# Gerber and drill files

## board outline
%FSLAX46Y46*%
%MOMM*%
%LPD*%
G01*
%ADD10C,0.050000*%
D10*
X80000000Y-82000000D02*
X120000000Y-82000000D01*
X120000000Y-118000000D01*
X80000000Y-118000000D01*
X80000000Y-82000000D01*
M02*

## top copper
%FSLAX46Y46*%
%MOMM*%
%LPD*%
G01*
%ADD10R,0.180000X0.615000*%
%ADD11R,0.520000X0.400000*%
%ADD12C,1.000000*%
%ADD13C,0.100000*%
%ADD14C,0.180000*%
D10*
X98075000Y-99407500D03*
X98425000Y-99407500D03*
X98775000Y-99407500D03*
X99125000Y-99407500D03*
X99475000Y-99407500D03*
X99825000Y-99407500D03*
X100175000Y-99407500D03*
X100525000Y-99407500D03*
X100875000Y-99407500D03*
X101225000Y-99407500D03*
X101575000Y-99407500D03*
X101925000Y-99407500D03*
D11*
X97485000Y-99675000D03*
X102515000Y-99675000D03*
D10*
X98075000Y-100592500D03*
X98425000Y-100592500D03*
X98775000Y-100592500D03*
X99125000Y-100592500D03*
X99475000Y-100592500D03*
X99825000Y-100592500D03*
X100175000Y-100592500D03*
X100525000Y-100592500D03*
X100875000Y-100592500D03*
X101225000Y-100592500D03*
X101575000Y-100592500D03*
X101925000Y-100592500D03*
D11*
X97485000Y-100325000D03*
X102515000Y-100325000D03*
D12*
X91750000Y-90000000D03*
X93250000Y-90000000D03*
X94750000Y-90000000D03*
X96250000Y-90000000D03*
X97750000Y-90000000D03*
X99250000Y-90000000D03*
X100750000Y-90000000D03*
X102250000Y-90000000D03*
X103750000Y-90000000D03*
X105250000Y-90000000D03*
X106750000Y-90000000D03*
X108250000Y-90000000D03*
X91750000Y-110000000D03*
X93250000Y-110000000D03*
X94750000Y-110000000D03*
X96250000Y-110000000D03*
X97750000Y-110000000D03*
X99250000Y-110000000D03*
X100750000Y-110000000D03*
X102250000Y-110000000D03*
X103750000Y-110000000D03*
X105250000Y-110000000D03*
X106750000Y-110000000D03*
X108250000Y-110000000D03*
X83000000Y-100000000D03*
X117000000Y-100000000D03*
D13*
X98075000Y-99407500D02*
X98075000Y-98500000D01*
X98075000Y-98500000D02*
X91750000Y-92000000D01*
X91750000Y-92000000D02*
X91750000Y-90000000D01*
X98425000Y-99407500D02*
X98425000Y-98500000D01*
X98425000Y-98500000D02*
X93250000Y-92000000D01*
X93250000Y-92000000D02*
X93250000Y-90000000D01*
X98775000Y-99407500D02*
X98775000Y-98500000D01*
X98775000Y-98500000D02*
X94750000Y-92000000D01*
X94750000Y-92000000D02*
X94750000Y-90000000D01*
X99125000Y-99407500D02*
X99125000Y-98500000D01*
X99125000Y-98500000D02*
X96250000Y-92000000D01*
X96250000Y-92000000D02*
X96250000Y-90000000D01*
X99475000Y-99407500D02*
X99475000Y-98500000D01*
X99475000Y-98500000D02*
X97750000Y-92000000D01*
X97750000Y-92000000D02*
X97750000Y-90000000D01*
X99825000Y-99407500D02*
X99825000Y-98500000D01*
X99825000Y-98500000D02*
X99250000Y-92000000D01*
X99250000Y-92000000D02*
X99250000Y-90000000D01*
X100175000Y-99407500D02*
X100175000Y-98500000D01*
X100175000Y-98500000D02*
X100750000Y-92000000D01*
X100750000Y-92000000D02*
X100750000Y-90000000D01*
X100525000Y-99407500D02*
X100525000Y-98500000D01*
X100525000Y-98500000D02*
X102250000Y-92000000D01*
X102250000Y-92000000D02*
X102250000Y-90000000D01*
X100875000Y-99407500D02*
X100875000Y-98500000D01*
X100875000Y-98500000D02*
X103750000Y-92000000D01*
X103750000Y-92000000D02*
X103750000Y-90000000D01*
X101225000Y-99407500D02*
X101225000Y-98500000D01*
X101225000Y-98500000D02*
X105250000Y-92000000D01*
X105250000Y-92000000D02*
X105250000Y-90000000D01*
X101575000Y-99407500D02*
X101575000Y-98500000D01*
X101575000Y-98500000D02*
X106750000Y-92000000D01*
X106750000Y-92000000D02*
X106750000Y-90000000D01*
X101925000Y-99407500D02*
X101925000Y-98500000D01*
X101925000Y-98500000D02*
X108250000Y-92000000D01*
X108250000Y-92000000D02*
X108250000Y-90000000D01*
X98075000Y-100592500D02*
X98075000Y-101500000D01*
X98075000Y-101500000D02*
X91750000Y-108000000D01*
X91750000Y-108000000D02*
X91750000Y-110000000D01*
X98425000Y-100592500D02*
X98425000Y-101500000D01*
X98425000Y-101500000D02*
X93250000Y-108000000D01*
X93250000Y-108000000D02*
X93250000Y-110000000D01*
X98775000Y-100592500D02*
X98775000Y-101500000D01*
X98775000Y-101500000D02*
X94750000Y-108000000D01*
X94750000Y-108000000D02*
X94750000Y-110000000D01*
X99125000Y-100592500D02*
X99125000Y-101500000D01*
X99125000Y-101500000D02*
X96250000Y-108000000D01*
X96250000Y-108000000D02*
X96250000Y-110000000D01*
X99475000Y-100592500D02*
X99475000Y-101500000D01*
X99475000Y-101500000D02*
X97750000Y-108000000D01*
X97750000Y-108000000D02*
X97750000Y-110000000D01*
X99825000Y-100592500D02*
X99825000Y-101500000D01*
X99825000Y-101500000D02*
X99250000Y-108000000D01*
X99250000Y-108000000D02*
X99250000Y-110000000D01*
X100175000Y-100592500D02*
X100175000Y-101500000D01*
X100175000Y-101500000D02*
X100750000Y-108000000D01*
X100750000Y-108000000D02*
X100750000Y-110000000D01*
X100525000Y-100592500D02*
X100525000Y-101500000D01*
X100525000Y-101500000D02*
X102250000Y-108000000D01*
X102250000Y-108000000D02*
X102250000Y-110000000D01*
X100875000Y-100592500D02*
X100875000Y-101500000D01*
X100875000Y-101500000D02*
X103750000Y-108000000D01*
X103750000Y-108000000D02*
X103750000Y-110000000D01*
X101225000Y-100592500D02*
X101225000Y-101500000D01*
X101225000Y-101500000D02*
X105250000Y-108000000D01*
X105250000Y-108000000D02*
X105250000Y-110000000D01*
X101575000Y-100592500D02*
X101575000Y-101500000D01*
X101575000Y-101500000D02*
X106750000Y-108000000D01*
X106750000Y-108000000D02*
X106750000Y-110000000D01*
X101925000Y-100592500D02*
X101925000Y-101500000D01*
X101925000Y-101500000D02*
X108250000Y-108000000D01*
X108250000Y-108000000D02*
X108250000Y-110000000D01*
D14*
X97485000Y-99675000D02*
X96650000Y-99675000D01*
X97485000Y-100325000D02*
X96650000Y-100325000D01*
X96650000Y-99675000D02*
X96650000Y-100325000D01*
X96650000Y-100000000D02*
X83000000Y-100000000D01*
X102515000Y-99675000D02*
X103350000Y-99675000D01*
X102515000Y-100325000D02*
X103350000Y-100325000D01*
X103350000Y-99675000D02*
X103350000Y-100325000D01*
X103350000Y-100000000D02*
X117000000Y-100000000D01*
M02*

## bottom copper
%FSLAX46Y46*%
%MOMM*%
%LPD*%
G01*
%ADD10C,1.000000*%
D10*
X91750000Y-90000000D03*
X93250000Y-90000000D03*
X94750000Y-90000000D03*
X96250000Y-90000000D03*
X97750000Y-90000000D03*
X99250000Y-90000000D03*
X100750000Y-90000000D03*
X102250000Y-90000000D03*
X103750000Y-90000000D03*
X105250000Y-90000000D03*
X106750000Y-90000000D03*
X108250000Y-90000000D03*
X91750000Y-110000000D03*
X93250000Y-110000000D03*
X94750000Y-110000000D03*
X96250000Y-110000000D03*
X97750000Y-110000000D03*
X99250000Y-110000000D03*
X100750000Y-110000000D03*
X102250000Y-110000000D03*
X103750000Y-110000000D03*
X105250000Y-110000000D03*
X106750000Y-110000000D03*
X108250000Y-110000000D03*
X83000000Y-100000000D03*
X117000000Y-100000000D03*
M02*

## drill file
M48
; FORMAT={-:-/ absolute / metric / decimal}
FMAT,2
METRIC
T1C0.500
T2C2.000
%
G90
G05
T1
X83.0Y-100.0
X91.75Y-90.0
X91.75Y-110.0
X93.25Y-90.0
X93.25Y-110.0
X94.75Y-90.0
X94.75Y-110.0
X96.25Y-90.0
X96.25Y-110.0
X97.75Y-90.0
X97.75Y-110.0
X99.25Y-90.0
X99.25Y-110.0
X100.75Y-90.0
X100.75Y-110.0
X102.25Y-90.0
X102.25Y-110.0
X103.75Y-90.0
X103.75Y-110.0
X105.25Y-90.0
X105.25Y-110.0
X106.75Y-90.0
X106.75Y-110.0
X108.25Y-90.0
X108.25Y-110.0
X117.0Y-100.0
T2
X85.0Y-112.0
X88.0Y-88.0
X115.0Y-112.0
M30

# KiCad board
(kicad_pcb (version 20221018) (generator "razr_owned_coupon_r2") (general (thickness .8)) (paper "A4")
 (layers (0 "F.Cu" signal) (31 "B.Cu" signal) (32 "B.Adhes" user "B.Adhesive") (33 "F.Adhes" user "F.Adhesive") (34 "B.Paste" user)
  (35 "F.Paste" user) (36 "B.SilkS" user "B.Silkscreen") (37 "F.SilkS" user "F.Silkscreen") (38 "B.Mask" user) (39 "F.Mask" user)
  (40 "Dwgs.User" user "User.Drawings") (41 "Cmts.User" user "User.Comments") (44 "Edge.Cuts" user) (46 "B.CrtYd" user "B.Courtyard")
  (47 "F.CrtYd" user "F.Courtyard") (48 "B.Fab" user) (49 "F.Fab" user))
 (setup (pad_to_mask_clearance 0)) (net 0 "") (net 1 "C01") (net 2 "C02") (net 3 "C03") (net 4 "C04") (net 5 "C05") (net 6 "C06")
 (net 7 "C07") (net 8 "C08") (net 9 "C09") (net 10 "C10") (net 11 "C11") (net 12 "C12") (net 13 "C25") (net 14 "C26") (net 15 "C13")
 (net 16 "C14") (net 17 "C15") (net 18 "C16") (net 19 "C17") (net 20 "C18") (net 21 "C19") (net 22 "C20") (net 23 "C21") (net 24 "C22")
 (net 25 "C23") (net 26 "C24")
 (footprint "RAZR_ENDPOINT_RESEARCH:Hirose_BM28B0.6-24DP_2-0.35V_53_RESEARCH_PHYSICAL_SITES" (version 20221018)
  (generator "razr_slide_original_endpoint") (layer "F.Cu") (at 100 100)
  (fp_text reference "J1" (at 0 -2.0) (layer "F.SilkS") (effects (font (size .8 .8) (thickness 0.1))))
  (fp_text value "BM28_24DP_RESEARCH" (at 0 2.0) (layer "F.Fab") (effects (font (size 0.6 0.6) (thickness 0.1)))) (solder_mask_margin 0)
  (pad "S_NEG_00" smd rect (at -1.925 -0.5925) (size 0.18 0.615) (layers "F.Cu" "F.Mask") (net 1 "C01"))
  (pad "S_NEG_01" smd rect (at -1.575 -0.5925) (size 0.18 0.615) (layers "F.Cu" "F.Mask") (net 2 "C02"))
  (pad "S_NEG_02" smd rect (at -1.225 -0.5925) (size 0.18 0.615) (layers "F.Cu" "F.Mask") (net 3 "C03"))
  (pad "S_NEG_03" smd rect (at -0.875 -0.5925) (size 0.18 0.615) (layers "F.Cu" "F.Mask") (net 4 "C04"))
  (pad "S_NEG_04" smd rect (at -0.525 -0.5925) (size 0.18 0.615) (layers "F.Cu" "F.Mask") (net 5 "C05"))
  (pad "S_NEG_05" smd rect (at -0.175 -0.5925) (size 0.18 0.615) (layers "F.Cu" "F.Mask") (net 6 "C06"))
  (pad "S_NEG_06" smd rect (at 0.175 -0.5925) (size 0.18 0.615) (layers "F.Cu" "F.Mask") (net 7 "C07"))
  (pad "S_NEG_07" smd rect (at 0.525 -0.5925) (size 0.18 0.615) (layers "F.Cu" "F.Mask") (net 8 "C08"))
  (pad "S_NEG_08" smd rect (at 0.875 -0.5925) (size 0.18 0.615) (layers "F.Cu" "F.Mask") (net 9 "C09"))
  (pad "S_NEG_09" smd rect (at 1.225 -0.5925) (size 0.18 0.615) (layers "F.Cu" "F.Mask") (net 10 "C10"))
  (pad "S_NEG_10" smd rect (at 1.575 -0.5925) (size 0.18 0.615) (layers "F.Cu" "F.Mask") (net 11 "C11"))
  (pad "S_NEG_11" smd rect (at 1.925 -0.5925) (size 0.18 0.615) (layers "F.Cu" "F.Mask") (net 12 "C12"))
  (pad "P_L" smd rect (at -2.515 -0.325) (size 0.52 0.4) (layers "F.Cu" "F.Mask") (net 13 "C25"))
  (pad "P_R" smd rect (at 2.515 -0.325) (size 0.52 0.4) (layers "F.Cu" "F.Mask") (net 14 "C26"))
  (pad "S_POS_00" smd rect (at -1.925 0.5925) (size 0.18 0.615) (layers "F.Cu" "F.Mask") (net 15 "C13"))
  (pad "S_POS_01" smd rect (at -1.575 0.5925) (size 0.18 0.615) (layers "F.Cu" "F.Mask") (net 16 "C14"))
  (pad "S_POS_02" smd rect (at -1.225 0.5925) (size 0.18 0.615) (layers "F.Cu" "F.Mask") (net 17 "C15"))
  (pad "S_POS_03" smd rect (at -0.875 0.5925) (size 0.18 0.615) (layers "F.Cu" "F.Mask") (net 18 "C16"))
  (pad "S_POS_04" smd rect (at -0.525 0.5925) (size 0.18 0.615) (layers "F.Cu" "F.Mask") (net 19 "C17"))
  (pad "S_POS_05" smd rect (at -0.175 0.5925) (size 0.18 0.615) (layers "F.Cu" "F.Mask") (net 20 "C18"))
  (pad "S_POS_06" smd rect (at 0.175 0.5925) (size 0.18 0.615) (layers "F.Cu" "F.Mask") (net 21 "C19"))
  (pad "S_POS_07" smd rect (at 0.525 0.5925) (size 0.18 0.615) (layers "F.Cu" "F.Mask") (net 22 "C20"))
  (pad "S_POS_08" smd rect (at 0.875 0.5925) (size 0.18 0.615) (layers "F.Cu" "F.Mask") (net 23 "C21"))
  (pad "S_POS_09" smd rect (at 1.225 0.5925) (size 0.18 0.615) (layers "F.Cu" "F.Mask") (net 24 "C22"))
  (pad "S_POS_10" smd rect (at 1.575 0.5925) (size 0.18 0.615) (layers "F.Cu" "F.Mask") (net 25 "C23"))
  (pad "S_POS_11" smd rect (at 1.925 0.5925) (size 0.18 0.615) (layers "F.Cu" "F.Mask") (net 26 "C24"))
  (pad "P_L" smd rect (at -2.515 0.325) (size 0.52 0.4) (layers "F.Cu" "F.Mask") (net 13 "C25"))
  (pad "P_R" smd rect (at 2.515 0.325) (size 0.52 0.4) (layers "F.Cu" "F.Mask") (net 14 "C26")))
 (segment (start 98.075000 99.407500) (end 98.075000 98.500000) (width 0.1) (layer "F.Cu") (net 1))
 (segment (start 98.075000 98.500000) (end 91.750000 92.000000) (width 0.1) (layer "F.Cu") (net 1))
 (segment (start 91.750000 92.000000) (end 91.750000 90.000000) (width 0.1) (layer "F.Cu") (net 1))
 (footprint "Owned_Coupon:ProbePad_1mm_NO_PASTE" (layer "F.Cu") (at 91.75 90)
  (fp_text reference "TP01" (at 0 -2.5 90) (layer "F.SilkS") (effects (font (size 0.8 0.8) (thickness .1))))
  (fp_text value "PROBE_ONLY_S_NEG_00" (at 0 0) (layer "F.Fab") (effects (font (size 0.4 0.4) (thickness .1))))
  (pad "1" thru_hole circle (at 0 0) (size 1 1) (drill .5) (layers "*.Cu" "*.Mask") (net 1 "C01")))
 (segment (start 98.425000 99.407500) (end 98.425000 98.500000) (width 0.1) (layer "F.Cu") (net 2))
 (segment (start 98.425000 98.500000) (end 93.250000 92.000000) (width 0.1) (layer "F.Cu") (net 2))
 (segment (start 93.250000 92.000000) (end 93.250000 90.000000) (width 0.1) (layer "F.Cu") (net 2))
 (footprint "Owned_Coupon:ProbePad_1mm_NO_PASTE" (layer "F.Cu") (at 93.25 90)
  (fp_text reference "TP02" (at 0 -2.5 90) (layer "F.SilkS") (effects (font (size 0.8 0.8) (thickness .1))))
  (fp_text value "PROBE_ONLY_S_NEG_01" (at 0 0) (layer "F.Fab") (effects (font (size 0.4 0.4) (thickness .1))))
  (pad "1" thru_hole circle (at 0 0) (size 1 1) (drill .5) (layers "*.Cu" "*.Mask") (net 2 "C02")))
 (segment (start 98.775000 99.407500) (end 98.775000 98.500000) (width 0.1) (layer "F.Cu") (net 3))
 (segment (start 98.775000 98.500000) (end 94.750000 92.000000) (width 0.1) (layer "F.Cu") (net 3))
 (segment (start 94.750000 92.000000) (end 94.750000 90.000000) (width 0.1) (layer "F.Cu") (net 3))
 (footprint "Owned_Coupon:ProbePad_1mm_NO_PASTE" (layer "F.Cu") (at 94.75 90)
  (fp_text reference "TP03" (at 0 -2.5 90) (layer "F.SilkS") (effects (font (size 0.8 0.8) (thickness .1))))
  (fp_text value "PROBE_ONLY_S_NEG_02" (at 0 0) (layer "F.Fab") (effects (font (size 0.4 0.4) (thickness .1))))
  (pad "1" thru_hole circle (at 0 0) (size 1 1) (drill .5) (layers "*.Cu" "*.Mask") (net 3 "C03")))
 (segment (start 99.125000 99.407500) (end 99.125000 98.500000) (width 0.1) (layer "F.Cu") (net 4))
 (segment (start 99.125000 98.500000) (end 96.250000 92.000000) (width 0.1) (layer "F.Cu") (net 4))
 (segment (start 96.250000 92.000000) (end 96.250000 90.000000) (width 0.1) (layer "F.Cu") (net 4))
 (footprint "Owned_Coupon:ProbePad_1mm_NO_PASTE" (layer "F.Cu") (at 96.25 90)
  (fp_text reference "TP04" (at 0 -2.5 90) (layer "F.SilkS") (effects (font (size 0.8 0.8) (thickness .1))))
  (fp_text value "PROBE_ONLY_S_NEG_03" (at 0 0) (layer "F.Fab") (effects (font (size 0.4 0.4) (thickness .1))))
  (pad "1" thru_hole circle (at 0 0) (size 1 1) (drill .5) (layers "*.Cu" "*.Mask") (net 4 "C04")))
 (segment (start 99.475000 99.407500) (end 99.475000 98.500000) (width 0.1) (layer "F.Cu") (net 5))
 (segment (start 99.475000 98.500000) (end 97.750000 92.000000) (width 0.1) (layer "F.Cu") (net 5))
 (segment (start 97.750000 92.000000) (end 97.750000 90.000000) (width 0.1) (layer "F.Cu") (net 5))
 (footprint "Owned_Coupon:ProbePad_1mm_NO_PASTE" (layer "F.Cu") (at 97.75 90)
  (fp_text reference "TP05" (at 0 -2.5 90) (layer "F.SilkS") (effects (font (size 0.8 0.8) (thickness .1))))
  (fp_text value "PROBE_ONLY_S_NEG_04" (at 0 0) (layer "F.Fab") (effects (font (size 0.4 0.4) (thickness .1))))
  (pad "1" thru_hole circle (at 0 0) (size 1 1) (drill .5) (layers "*.Cu" "*.Mask") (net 5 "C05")))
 (segment (start 99.825000 99.407500) (end 99.825000 98.500000) (width 0.1) (layer "F.Cu") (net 6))
 (segment (start 99.825000 98.500000) (end 99.250000 92.000000) (width 0.1) (layer "F.Cu") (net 6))
 (segment (start 99.250000 92.000000) (end 99.250000 90.000000) (width 0.1) (layer "F.Cu") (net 6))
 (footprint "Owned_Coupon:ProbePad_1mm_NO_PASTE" (layer "F.Cu") (at 99.25 90)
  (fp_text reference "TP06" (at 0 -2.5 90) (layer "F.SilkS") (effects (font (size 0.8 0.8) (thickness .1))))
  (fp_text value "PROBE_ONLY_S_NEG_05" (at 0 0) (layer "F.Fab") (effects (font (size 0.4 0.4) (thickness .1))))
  (pad "1" thru_hole circle (at 0 0) (size 1 1) (drill .5) (layers "*.Cu" "*.Mask") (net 6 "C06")))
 (segment (start 100.175000 99.407500) (end 100.175000 98.500000) (width 0.1) (layer "F.Cu") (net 7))
 (segment (start 100.175000 98.500000) (end 100.750000 92.000000) (width 0.1) (layer "F.Cu") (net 7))
 (segment (start 100.750000 92.000000) (end 100.750000 90.000000) (width 0.1) (layer "F.Cu") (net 7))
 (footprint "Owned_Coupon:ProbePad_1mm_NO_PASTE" (layer "F.Cu") (at 100.75 90)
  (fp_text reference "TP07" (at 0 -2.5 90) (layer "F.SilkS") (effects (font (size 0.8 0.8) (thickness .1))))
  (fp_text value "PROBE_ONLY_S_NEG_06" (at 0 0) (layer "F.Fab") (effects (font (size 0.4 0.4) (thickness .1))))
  (pad "1" thru_hole circle (at 0 0) (size 1 1) (drill .5) (layers "*.Cu" "*.Mask") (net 7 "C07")))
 (segment (start 100.525000 99.407500) (end 100.525000 98.500000) (width 0.1) (layer "F.Cu") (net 8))
 (segment (start 100.525000 98.500000) (end 102.250000 92.000000) (width 0.1) (layer "F.Cu") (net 8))
 (segment (start 102.250000 92.000000) (end 102.250000 90.000000) (width 0.1) (layer "F.Cu") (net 8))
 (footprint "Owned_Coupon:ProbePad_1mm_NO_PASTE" (layer "F.Cu") (at 102.25 90)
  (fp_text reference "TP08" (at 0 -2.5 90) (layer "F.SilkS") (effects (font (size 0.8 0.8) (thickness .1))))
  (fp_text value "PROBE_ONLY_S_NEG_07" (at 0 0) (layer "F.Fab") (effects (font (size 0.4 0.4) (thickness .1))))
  (pad "1" thru_hole circle (at 0 0) (size 1 1) (drill .5) (layers "*.Cu" "*.Mask") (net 8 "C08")))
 (segment (start 100.875000 99.407500) (end 100.875000 98.500000) (width 0.1) (layer "F.Cu") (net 9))
 (segment (start 100.875000 98.500000) (end 103.750000 92.000000) (width 0.1) (layer "F.Cu") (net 9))
 (segment (start 103.750000 92.000000) (end 103.750000 90.000000) (width 0.1) (layer "F.Cu") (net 9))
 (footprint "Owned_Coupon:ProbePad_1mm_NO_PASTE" (layer "F.Cu") (at 103.75 90)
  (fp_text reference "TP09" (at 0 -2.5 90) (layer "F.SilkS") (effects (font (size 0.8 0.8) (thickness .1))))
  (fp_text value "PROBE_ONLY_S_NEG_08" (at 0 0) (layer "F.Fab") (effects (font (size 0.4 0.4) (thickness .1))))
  (pad "1" thru_hole circle (at 0 0) (size 1 1) (drill .5) (layers "*.Cu" "*.Mask") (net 9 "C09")))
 (segment (start 101.225000 99.407500) (end 101.225000 98.500000) (width 0.1) (layer "F.Cu") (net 10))
 (segment (start 101.225000 98.500000) (end 105.250000 92.000000) (width 0.1) (layer "F.Cu") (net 10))
 (segment (start 105.250000 92.000000) (end 105.250000 90.000000) (width 0.1) (layer "F.Cu") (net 10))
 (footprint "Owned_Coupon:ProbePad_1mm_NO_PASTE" (layer "F.Cu") (at 105.25 90)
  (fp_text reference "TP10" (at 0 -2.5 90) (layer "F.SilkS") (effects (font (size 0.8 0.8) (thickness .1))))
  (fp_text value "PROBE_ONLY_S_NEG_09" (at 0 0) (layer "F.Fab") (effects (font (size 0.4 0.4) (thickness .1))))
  (pad "1" thru_hole circle (at 0 0) (size 1 1) (drill .5) (layers "*.Cu" "*.Mask") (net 10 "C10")))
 (segment (start 101.575000 99.407500) (end 101.575000 98.500000) (width 0.1) (layer "F.Cu") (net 11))
 (segment (start 101.575000 98.500000) (end 106.750000 92.000000) (width 0.1) (layer "F.Cu") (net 11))
 (segment (start 106.750000 92.000000) (end 106.750000 90.000000) (width 0.1) (layer "F.Cu") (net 11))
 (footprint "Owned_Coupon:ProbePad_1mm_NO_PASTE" (layer "F.Cu") (at 106.75 90)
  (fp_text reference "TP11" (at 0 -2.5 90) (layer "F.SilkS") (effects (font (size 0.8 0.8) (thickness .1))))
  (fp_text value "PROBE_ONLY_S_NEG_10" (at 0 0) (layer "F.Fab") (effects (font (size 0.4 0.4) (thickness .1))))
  (pad "1" thru_hole circle (at 0 0) (size 1 1) (drill .5) (layers "*.Cu" "*.Mask") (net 11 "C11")))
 (segment (start 101.925000 99.407500) (end 101.925000 98.500000) (width 0.1) (layer "F.Cu") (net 12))
 (segment (start 101.925000 98.500000) (end 108.250000 92.000000) (width 0.1) (layer "F.Cu") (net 12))
 (segment (start 108.250000 92.000000) (end 108.250000 90.000000) (width 0.1) (layer "F.Cu") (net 12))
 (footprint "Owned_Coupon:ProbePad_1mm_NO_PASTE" (layer "F.Cu") (at 108.25 90)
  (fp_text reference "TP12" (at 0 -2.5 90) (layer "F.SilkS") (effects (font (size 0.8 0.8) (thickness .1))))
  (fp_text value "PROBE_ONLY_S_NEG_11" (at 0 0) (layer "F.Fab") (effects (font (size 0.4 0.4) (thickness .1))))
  (pad "1" thru_hole circle (at 0 0) (size 1 1) (drill .5) (layers "*.Cu" "*.Mask") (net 12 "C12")))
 (segment (start 98.075000 100.592500) (end 98.075000 101.500000) (width 0.1) (layer "F.Cu") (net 15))
 (segment (start 98.075000 101.500000) (end 91.750000 108.000000) (width 0.1) (layer "F.Cu") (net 15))
 (segment (start 91.750000 108.000000) (end 91.750000 110.000000) (width 0.1) (layer "F.Cu") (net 15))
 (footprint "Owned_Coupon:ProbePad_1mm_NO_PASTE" (layer "F.Cu") (at 91.75 110)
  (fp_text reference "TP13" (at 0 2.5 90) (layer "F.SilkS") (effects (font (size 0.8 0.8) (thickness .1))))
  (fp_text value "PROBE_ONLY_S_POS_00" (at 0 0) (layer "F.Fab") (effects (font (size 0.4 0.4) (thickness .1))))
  (pad "1" thru_hole circle (at 0 0) (size 1 1) (drill .5) (layers "*.Cu" "*.Mask") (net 15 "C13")))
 (segment (start 98.425000 100.592500) (end 98.425000 101.500000) (width 0.1) (layer "F.Cu") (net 16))
 (segment (start 98.425000 101.500000) (end 93.250000 108.000000) (width 0.1) (layer "F.Cu") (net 16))
 (segment (start 93.250000 108.000000) (end 93.250000 110.000000) (width 0.1) (layer "F.Cu") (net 16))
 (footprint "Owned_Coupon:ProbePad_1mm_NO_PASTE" (layer "F.Cu") (at 93.25 110)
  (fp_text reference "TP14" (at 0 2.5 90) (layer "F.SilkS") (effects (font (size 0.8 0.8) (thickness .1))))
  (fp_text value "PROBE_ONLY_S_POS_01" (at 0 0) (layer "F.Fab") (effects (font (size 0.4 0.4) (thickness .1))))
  (pad "1" thru_hole circle (at 0 0) (size 1 1) (drill .5) (layers "*.Cu" "*.Mask") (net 16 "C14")))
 (segment (start 98.775000 100.592500) (end 98.775000 101.500000) (width 0.1) (layer "F.Cu") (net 17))
 (segment (start 98.775000 101.500000) (end 94.750000 108.000000) (width 0.1) (layer "F.Cu") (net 17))
 (segment (start 94.750000 108.000000) (end 94.750000 110.000000) (width 0.1) (layer "F.Cu") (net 17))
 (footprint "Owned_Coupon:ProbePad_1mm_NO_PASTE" (layer "F.Cu") (at 94.75 110)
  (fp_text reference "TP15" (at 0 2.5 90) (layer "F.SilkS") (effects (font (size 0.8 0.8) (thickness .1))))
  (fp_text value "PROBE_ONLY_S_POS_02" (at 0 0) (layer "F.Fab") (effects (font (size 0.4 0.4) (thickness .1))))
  (pad "1" thru_hole circle (at 0 0) (size 1 1) (drill .5) (layers "*.Cu" "*.Mask") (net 17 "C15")))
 (segment (start 99.125000 100.592500) (end 99.125000 101.500000) (width 0.1) (layer "F.Cu") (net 18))
 (segment (start 99.125000 101.500000) (end 96.250000 108.000000) (width 0.1) (layer "F.Cu") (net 18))
 (segment (start 96.250000 108.000000) (end 96.250000 110.000000) (width 0.1) (layer "F.Cu") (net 18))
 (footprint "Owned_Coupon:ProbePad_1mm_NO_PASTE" (layer "F.Cu") (at 96.25 110)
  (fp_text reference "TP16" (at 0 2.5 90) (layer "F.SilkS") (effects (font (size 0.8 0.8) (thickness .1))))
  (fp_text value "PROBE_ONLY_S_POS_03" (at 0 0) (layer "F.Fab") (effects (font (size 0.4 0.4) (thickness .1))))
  (pad "1" thru_hole circle (at 0 0) (size 1 1) (drill .5) (layers "*.Cu" "*.Mask") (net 18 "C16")))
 (segment (start 99.475000 100.592500) (end 99.475000 101.500000) (width 0.1) (layer "F.Cu") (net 19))
 (segment (start 99.475000 101.500000) (end 97.750000 108.000000) (width 0.1) (layer "F.Cu") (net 19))
 (segment (start 97.750000 108.000000) (end 97.750000 110.000000) (width 0.1) (layer "F.Cu") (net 19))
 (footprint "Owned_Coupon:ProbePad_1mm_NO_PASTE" (layer "F.Cu") (at 97.75 110)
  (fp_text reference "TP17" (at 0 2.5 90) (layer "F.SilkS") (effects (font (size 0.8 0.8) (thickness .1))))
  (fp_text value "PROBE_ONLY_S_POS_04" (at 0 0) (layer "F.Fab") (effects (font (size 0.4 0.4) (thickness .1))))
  (pad "1" thru_hole circle (at 0 0) (size 1 1) (drill .5) (layers "*.Cu" "*.Mask") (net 19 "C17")))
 (segment (start 99.825000 100.592500) (end 99.825000 101.500000) (width 0.1) (layer "F.Cu") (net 20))
 (segment (start 99.825000 101.500000) (end 99.250000 108.000000) (width 0.1) (layer "F.Cu") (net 20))
 (segment (start 99.250000 108.000000) (end 99.250000 110.000000) (width 0.1) (layer "F.Cu") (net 20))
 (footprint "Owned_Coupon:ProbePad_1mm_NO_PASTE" (layer "F.Cu") (at 99.25 110)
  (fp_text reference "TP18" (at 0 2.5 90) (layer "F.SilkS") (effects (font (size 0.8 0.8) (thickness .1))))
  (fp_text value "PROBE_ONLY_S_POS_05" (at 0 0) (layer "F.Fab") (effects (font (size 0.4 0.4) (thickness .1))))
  (pad "1" thru_hole circle (at 0 0) (size 1 1) (drill .5) (layers "*.Cu" "*.Mask") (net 20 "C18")))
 (segment (start 100.175000 100.592500) (end 100.175000 101.500000) (width 0.1) (layer "F.Cu") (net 21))
 (segment (start 100.175000 101.500000) (end 100.750000 108.000000) (width 0.1) (layer "F.Cu") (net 21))
 (segment (start 100.750000 108.000000) (end 100.750000 110.000000) (width 0.1) (layer "F.Cu") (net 21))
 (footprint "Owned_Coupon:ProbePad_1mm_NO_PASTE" (layer "F.Cu") (at 100.75 110)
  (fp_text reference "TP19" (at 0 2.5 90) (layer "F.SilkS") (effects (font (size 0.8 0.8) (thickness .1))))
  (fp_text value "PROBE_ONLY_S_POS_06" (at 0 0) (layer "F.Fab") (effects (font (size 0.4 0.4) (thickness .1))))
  (pad "1" thru_hole circle (at 0 0) (size 1 1) (drill .5) (layers "*.Cu" "*.Mask") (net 21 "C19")))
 (segment (start 100.525000 100.592500) (end 100.525000 101.500000) (width 0.1) (layer "F.Cu") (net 22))
 (segment (start 100.525000 101.500000) (end 102.250000 108.000000) (width 0.1) (layer "F.Cu") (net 22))
 (segment (start 102.250000 108.000000) (end 102.250000 110.000000) (width 0.1) (layer "F.Cu") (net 22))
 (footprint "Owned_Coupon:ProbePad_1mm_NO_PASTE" (layer "F.Cu") (at 102.25 110)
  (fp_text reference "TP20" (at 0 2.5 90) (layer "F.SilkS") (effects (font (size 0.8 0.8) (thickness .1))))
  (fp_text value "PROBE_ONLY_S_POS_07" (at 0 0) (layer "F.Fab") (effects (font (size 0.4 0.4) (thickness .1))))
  (pad "1" thru_hole circle (at 0 0) (size 1 1) (drill .5) (layers "*.Cu" "*.Mask") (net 22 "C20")))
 (segment (start 100.875000 100.592500) (end 100.875000 101.500000) (width 0.1) (layer "F.Cu") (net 23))
 (segment (start 100.875000 101.500000) (end 103.750000 108.000000) (width 0.1) (layer "F.Cu") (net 23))
 (segment (start 103.750000 108.000000) (end 103.750000 110.000000) (width 0.1) (layer "F.Cu") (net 23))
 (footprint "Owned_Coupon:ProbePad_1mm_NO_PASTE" (layer "F.Cu") (at 103.75 110)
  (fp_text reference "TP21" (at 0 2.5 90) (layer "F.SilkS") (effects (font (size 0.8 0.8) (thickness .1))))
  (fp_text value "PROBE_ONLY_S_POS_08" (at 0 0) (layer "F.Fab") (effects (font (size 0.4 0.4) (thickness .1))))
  (pad "1" thru_hole circle (at 0 0) (size 1 1) (drill .5) (layers "*.Cu" "*.Mask") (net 23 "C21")))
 (segment (start 101.225000 100.592500) (end 101.225000 101.500000) (width 0.1) (layer "F.Cu") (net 24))
 (segment (start 101.225000 101.500000) (end 105.250000 108.000000) (width 0.1) (layer "F.Cu") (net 24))
 (segment (start 105.250000 108.000000) (end 105.250000 110.000000) (width 0.1) (layer "F.Cu") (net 24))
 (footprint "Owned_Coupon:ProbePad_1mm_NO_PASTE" (layer "F.Cu") (at 105.25 110)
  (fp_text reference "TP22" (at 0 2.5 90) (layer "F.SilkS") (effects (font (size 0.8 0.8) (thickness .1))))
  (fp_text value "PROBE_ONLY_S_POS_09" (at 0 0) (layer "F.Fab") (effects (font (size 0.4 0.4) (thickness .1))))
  (pad "1" thru_hole circle (at 0 0) (size 1 1) (drill .5) (layers "*.Cu" "*.Mask") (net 24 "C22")))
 (segment (start 101.575000 100.592500) (end 101.575000 101.500000) (width 0.1) (layer "F.Cu") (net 25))
 (segment (start 101.575000 101.500000) (end 106.750000 108.000000) (width 0.1) (layer "F.Cu") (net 25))
 (segment (start 106.750000 108.000000) (end 106.750000 110.000000) (width 0.1) (layer "F.Cu") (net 25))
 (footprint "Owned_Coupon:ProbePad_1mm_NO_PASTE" (layer "F.Cu") (at 106.75 110)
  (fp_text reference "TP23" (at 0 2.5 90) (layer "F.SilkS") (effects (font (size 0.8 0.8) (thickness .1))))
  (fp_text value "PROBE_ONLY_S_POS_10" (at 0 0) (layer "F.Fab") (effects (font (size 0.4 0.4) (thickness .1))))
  (pad "1" thru_hole circle (at 0 0) (size 1 1) (drill .5) (layers "*.Cu" "*.Mask") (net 25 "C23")))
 (segment (start 101.925000 100.592500) (end 101.925000 101.500000) (width 0.1) (layer "F.Cu") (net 26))
 (segment (start 101.925000 101.500000) (end 108.250000 108.000000) (width 0.1) (layer "F.Cu") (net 26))
 (segment (start 108.250000 108.000000) (end 108.250000 110.000000) (width 0.1) (layer "F.Cu") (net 26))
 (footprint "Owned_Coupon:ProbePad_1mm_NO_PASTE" (layer "F.Cu") (at 108.25 110)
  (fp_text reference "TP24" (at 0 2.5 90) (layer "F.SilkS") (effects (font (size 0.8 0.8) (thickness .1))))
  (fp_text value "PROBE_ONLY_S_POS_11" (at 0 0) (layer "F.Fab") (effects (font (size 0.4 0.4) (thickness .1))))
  (pad "1" thru_hole circle (at 0 0) (size 1 1) (drill .5) (layers "*.Cu" "*.Mask") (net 26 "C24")))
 (segment (start 97.485000 99.675000) (end 96.650000 99.675000) (width 0.18) (layer "F.Cu") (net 13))
 (segment (start 97.485000 100.325000) (end 96.650000 100.325000) (width 0.18) (layer "F.Cu") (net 13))
 (segment (start 96.650000 99.675000) (end 96.650000 100.325000) (width 0.18) (layer "F.Cu") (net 13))
 (segment (start 96.650000 100.000000) (end 83.000000 100.000000) (width 0.18) (layer "F.Cu") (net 13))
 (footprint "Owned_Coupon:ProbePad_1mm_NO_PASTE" (layer "F.Cu") (at 83 100)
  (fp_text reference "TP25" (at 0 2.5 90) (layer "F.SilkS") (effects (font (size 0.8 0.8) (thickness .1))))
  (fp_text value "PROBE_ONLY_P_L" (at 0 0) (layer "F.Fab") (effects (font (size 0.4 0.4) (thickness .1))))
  (pad "1" thru_hole circle (at 0 0) (size 1 1) (drill .5) (layers "*.Cu" "*.Mask") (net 13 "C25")))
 (segment (start 102.515000 99.675000) (end 103.350000 99.675000) (width 0.18) (layer "F.Cu") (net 14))
 (segment (start 102.515000 100.325000) (end 103.350000 100.325000) (width 0.18) (layer "F.Cu") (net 14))
 (segment (start 103.350000 99.675000) (end 103.350000 100.325000) (width 0.18) (layer "F.Cu") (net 14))
 (segment (start 103.350000 100.000000) (end 117.000000 100.000000) (width 0.18) (layer "F.Cu") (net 14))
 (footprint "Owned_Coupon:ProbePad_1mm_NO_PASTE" (layer "F.Cu") (at 117 100)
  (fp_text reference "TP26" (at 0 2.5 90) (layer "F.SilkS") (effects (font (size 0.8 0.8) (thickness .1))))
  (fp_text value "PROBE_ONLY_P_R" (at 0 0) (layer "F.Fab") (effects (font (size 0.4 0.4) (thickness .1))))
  (pad "1" thru_hole circle (at 0 0) (size 1 1) (drill .5) (layers "*.Cu" "*.Mask") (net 14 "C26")))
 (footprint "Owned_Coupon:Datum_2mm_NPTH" (layer "F.Cu") (at 85 112)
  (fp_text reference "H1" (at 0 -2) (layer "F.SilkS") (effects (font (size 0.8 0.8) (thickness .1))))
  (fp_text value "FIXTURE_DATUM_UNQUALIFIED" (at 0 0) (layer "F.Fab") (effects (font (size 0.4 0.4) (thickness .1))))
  (pad "" np_thru_hole circle (at 0 0) (size 2 2) (drill 2) (layers "*.Cu" "*.Mask")))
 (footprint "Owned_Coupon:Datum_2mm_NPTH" (layer "F.Cu") (at 115 112)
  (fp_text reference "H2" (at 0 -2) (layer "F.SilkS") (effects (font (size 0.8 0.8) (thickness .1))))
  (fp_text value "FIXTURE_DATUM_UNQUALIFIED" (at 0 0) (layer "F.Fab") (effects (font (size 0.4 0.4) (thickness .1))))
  (pad "" np_thru_hole circle (at 0 0) (size 2 2) (drill 2) (layers "*.Cu" "*.Mask")))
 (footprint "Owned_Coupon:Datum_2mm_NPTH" (layer "F.Cu") (at 88 88)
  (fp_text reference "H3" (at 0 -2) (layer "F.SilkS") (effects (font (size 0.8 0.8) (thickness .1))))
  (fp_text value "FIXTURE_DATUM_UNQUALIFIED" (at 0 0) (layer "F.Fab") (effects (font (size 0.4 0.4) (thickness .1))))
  (pad "" np_thru_hole circle (at 0 0) (size 2 2) (drill 2) (layers "*.Cu" "*.Mask")))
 (gr_rect (start 80 82) (end 120 118) (stroke (width .05) (type default)) (fill none) (layer "Edge.Cuts")))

